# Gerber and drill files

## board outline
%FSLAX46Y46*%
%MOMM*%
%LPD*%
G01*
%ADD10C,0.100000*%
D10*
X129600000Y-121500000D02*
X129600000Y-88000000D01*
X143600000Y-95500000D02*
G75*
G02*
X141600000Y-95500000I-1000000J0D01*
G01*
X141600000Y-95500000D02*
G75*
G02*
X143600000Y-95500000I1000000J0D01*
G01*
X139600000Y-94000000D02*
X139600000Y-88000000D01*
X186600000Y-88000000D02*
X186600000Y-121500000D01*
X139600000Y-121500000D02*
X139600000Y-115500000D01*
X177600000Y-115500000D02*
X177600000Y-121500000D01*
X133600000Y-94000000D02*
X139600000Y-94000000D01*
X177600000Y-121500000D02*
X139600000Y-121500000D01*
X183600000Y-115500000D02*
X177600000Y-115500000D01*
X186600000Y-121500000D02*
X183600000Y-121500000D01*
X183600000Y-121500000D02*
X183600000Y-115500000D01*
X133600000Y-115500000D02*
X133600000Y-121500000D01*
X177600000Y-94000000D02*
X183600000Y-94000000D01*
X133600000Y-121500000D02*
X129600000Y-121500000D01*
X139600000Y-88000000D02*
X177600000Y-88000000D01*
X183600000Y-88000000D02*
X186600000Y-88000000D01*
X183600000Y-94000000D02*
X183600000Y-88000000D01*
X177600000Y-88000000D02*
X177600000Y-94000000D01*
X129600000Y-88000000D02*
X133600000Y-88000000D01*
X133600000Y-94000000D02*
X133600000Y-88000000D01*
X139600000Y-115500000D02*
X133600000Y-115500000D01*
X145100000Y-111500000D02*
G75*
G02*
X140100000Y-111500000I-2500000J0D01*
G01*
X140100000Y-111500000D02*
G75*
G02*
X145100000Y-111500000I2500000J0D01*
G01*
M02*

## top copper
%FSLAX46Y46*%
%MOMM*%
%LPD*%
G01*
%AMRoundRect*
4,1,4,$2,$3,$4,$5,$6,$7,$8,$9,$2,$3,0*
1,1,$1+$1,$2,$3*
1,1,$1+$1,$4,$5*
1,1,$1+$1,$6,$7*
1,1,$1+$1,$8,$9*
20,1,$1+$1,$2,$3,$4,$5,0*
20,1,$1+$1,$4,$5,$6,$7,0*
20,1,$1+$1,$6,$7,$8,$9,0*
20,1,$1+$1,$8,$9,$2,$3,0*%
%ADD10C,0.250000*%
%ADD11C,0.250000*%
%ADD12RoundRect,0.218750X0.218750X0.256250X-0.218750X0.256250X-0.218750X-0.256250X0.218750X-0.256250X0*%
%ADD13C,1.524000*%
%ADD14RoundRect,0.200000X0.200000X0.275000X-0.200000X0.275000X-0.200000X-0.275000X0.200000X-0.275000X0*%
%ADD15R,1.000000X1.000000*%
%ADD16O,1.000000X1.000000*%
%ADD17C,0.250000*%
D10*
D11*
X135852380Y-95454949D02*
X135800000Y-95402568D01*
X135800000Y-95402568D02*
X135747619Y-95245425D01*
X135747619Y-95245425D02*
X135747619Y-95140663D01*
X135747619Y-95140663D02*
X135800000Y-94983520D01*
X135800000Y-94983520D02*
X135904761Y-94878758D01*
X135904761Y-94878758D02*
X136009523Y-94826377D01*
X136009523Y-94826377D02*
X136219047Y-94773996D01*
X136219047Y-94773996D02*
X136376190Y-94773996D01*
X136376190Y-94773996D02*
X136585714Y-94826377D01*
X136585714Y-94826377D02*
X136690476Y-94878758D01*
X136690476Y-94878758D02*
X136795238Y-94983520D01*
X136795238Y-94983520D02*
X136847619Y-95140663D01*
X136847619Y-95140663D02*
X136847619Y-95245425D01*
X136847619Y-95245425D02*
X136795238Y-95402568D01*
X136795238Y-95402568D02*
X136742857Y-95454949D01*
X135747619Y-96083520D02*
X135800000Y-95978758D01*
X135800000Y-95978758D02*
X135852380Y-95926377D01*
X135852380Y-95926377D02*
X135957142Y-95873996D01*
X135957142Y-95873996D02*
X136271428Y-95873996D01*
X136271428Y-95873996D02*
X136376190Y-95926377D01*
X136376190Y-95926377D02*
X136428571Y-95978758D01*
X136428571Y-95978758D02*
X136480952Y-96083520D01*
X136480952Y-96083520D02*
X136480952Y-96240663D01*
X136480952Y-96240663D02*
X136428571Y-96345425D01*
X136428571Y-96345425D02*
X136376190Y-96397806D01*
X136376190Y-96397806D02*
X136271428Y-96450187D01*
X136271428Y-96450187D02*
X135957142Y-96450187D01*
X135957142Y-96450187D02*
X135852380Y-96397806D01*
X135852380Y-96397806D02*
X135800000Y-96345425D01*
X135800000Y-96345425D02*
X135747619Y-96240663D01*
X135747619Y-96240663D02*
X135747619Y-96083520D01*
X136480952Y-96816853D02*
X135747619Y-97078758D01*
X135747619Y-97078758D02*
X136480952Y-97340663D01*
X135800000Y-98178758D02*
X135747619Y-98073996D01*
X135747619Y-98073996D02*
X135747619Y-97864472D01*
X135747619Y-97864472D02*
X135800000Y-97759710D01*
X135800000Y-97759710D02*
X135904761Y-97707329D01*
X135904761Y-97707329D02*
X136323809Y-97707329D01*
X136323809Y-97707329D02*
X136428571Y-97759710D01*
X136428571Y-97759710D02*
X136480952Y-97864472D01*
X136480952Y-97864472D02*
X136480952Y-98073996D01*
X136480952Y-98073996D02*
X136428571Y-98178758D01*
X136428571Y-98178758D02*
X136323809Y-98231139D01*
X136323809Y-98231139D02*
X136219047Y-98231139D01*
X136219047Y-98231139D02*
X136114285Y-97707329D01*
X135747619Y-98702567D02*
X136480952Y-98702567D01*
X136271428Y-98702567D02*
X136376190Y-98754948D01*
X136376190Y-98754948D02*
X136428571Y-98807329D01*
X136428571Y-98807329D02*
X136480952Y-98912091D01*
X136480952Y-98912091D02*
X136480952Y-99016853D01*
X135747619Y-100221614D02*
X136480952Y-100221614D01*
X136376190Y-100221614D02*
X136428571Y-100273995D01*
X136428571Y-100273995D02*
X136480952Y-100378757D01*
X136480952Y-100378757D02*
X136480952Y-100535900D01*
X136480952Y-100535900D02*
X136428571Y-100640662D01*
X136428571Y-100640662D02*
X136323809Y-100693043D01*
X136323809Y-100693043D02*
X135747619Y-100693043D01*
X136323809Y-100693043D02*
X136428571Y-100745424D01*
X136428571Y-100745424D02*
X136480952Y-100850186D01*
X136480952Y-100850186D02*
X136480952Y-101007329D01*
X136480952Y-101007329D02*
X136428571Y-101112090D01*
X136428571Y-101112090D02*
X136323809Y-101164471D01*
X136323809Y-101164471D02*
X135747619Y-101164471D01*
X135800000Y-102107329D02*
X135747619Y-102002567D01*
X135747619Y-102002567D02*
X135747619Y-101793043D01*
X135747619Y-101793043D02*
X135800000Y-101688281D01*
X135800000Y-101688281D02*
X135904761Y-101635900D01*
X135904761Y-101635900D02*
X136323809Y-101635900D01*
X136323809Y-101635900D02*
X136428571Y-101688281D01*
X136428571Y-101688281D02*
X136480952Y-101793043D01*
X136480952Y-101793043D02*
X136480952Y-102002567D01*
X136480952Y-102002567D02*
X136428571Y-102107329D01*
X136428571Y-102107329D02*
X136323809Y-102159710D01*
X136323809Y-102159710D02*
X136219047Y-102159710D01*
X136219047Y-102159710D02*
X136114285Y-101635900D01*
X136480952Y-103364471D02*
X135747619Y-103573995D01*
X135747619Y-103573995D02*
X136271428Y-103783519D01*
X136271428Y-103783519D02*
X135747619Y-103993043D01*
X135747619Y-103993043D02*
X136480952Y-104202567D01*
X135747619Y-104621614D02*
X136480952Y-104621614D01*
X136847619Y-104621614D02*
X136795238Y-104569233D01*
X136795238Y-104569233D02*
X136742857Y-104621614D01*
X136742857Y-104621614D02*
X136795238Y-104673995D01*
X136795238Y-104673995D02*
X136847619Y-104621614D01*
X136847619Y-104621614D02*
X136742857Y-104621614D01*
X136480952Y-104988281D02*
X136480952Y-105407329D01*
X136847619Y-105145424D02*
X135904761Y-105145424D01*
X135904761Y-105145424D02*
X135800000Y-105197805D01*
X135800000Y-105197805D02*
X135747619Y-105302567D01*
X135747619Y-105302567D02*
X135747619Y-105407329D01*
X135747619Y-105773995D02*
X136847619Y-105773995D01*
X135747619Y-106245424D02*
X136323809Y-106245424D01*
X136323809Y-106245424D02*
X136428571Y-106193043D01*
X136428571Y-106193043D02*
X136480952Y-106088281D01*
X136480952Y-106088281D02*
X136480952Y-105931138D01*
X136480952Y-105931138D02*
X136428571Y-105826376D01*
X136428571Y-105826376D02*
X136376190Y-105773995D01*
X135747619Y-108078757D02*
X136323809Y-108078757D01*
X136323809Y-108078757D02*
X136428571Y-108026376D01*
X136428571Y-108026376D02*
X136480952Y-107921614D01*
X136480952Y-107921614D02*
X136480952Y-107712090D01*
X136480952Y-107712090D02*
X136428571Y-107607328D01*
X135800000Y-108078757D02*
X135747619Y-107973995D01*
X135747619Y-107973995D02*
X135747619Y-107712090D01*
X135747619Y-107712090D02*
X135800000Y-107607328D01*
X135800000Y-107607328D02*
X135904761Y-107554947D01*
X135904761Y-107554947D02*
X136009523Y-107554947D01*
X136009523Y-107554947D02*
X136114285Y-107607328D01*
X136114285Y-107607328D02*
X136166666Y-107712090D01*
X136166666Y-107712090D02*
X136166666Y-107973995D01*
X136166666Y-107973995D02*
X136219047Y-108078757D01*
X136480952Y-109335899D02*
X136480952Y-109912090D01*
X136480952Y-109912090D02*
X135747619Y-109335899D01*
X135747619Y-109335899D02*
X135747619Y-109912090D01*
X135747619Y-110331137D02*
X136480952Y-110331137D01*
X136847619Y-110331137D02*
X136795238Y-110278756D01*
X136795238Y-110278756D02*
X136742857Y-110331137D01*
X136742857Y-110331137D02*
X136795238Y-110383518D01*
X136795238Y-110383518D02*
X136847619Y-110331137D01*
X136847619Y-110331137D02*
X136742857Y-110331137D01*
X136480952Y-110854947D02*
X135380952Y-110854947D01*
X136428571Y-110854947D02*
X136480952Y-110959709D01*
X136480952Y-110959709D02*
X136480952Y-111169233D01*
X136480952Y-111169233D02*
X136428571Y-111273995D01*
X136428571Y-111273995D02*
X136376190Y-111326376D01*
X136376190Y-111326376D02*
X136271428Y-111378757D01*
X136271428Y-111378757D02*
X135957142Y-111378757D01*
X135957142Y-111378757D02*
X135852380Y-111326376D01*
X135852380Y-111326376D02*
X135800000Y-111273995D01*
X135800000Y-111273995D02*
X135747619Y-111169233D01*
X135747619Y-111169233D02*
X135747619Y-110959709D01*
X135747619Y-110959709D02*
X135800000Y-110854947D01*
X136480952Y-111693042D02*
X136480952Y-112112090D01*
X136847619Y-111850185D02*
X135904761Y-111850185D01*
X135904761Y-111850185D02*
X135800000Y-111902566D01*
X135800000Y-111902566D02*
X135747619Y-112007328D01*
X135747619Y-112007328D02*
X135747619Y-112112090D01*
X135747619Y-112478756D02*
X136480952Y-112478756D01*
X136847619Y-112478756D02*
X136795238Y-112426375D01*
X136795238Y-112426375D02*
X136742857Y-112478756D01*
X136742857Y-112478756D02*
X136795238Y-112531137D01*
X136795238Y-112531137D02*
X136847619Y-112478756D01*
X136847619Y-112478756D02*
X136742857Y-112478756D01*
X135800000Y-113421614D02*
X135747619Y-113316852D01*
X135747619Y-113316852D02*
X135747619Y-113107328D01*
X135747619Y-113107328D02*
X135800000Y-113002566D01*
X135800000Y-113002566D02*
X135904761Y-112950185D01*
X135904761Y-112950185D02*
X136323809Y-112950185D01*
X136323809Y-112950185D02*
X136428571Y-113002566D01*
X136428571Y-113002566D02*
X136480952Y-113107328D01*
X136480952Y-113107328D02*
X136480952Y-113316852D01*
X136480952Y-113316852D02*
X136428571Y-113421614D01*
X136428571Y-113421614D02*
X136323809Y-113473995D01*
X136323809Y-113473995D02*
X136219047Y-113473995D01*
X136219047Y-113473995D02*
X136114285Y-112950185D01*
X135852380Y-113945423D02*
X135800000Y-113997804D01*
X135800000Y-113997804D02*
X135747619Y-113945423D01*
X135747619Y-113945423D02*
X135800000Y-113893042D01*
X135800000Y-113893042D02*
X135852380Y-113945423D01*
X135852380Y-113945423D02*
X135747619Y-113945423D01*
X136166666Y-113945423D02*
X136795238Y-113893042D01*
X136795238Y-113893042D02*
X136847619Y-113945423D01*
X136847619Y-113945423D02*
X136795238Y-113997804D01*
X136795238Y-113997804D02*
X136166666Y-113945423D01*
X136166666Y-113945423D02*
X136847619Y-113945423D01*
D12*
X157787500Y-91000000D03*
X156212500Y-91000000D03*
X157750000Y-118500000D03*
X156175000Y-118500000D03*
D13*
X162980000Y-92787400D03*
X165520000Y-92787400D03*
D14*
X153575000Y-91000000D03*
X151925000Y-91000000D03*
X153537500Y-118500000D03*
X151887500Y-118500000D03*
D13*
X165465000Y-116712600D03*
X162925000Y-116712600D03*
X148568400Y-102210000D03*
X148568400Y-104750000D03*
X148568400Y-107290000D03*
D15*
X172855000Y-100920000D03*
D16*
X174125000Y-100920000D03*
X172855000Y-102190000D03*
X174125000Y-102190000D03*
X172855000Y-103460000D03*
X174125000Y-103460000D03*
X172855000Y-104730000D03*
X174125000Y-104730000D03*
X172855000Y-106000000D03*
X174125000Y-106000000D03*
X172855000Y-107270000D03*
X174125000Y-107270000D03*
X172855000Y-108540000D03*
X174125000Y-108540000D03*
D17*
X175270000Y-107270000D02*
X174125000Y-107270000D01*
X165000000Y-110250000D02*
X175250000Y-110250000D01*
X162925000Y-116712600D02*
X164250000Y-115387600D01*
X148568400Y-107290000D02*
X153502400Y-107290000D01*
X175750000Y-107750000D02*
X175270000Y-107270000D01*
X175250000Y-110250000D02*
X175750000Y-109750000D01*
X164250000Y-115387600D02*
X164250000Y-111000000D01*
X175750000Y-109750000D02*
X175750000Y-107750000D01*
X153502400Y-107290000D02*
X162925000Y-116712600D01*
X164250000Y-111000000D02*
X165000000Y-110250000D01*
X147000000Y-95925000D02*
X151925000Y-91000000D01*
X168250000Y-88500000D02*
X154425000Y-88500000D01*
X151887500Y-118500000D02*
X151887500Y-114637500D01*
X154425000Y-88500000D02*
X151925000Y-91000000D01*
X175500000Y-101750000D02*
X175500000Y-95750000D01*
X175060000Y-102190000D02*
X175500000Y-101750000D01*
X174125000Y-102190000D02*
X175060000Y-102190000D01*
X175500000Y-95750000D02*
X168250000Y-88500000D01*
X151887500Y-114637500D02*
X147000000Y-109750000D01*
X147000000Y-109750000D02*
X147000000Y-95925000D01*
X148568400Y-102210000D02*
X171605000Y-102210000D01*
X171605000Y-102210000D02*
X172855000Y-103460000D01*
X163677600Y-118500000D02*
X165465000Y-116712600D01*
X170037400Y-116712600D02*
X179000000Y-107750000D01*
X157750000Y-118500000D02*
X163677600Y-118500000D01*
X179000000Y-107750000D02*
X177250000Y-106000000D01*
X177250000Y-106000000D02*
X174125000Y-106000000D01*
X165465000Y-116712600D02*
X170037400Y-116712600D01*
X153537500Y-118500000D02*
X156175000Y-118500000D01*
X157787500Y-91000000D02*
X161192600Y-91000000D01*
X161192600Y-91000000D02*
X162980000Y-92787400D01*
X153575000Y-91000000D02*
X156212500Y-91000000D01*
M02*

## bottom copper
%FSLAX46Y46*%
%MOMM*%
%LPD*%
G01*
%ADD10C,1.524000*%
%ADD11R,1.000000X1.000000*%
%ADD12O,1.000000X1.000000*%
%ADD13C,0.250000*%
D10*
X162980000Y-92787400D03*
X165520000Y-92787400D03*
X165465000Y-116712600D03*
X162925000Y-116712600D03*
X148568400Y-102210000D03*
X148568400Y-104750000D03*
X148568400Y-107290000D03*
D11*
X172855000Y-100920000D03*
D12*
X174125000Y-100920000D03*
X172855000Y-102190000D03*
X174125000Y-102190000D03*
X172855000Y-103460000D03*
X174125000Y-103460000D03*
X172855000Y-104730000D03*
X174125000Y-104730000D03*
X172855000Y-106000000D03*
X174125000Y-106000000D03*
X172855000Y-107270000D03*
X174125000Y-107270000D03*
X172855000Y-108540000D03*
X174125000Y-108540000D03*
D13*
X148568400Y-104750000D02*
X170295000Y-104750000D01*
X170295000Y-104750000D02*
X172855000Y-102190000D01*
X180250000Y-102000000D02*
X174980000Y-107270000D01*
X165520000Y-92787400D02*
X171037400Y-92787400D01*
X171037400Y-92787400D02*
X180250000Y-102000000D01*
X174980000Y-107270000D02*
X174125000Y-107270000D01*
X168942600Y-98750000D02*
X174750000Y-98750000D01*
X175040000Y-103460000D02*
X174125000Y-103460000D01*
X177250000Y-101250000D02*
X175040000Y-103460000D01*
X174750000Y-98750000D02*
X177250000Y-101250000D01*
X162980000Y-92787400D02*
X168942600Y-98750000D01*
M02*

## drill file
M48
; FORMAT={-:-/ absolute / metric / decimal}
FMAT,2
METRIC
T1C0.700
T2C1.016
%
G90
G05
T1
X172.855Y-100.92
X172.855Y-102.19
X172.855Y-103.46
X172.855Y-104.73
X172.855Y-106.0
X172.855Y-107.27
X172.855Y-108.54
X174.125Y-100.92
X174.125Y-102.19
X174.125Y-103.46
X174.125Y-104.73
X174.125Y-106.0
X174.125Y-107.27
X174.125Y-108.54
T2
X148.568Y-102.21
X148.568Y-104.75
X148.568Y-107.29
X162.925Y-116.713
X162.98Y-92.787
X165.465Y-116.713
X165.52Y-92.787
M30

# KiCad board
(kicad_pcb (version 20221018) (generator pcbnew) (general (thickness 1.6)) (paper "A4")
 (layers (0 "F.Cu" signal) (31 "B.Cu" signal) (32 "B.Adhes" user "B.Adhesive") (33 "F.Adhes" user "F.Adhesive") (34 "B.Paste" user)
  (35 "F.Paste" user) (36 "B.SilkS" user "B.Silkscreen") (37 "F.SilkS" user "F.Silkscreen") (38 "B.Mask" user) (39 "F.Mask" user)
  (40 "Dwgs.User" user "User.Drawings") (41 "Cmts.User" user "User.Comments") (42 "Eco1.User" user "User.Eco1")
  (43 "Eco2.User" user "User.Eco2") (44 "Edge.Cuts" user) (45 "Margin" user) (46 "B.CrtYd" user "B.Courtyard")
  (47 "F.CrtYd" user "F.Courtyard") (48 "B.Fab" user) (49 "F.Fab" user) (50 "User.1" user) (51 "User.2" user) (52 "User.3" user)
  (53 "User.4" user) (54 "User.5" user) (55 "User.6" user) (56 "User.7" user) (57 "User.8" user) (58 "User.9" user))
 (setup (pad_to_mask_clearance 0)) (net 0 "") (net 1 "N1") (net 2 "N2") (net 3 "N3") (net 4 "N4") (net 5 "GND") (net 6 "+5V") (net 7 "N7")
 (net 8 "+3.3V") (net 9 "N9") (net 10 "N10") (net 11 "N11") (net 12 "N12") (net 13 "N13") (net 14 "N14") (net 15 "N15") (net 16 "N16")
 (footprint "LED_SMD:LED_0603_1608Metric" (layer "F.Cu") (at 157 91 180)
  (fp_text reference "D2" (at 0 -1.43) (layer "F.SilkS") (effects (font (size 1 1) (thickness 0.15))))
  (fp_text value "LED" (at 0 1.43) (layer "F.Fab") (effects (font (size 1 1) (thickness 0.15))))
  (pad "1" smd roundrect (at -0.7875 0 180) (size 0.875 0.95) (layers "F.Cu" "F.Paste" "F.Mask") (roundrect_rratio 0.25) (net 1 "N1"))
  (pad "2" smd roundrect (at 0.7875 0 180) (size 0.875 0.95) (layers "F.Cu" "F.Paste" "F.Mask") (roundrect_rratio 0.25) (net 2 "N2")))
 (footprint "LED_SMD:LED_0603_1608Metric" (layer "F.Cu") (at 156.9625 118.5 180)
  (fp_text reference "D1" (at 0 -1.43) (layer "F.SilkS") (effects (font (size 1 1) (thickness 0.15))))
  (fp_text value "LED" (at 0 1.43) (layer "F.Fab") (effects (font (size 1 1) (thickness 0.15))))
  (pad "1" smd roundrect (at -0.7875 0 180) (size 0.875 0.95) (layers "F.Cu" "F.Paste" "F.Mask") (roundrect_rratio 0.25) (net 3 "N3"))
  (pad "2" smd roundrect (at 0.7875 0 180) (size 0.875 0.95) (layers "F.Cu" "F.Paste" "F.Mask") (roundrect_rratio 0.25) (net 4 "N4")))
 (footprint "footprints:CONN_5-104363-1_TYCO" (layer "F.Cu") (at 162.98 92.7874)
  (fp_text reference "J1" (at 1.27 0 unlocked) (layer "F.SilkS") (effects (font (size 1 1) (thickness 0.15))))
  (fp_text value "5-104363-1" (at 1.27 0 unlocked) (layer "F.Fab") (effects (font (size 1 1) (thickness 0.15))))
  (pad "1" thru_hole circle (at 0 0) (size 1.524 1.524) (drill 1.016) (layers "*.Cu" "*.Mask") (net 1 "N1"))
  (pad "2" thru_hole circle (at 2.54 0) (size 1.524 1.524) (drill 1.016) (layers "*.Cu" "*.Mask") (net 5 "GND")))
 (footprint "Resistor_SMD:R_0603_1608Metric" (layer "F.Cu") (at 152.75 91 180)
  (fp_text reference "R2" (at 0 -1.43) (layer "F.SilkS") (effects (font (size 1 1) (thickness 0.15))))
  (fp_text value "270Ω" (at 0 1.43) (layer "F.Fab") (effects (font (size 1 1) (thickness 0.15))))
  (pad "1" smd roundrect (at -0.825 0 180) (size 0.8 0.95) (layers "F.Cu" "F.Paste" "F.Mask") (roundrect_rratio 0.25) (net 2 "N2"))
  (pad "2" smd roundrect (at 0.825 0 180) (size 0.8 0.95) (layers "F.Cu" "F.Paste" "F.Mask") (roundrect_rratio 0.25) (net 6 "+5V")))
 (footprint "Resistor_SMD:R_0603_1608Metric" (layer "F.Cu") (at 152.7125 118.5 180)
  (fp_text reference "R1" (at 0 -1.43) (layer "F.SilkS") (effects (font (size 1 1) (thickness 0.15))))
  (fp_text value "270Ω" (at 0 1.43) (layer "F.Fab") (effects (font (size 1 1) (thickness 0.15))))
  (pad "1" smd roundrect (at -0.825 0 180) (size 0.8 0.95) (layers "F.Cu" "F.Paste" "F.Mask") (roundrect_rratio 0.25) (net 4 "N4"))
  (pad "2" smd roundrect (at 0.825 0 180) (size 0.8 0.95) (layers "F.Cu" "F.Paste" "F.Mask") (roundrect_rratio 0.25) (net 6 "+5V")))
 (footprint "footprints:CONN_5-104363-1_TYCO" (layer "F.Cu") (at 165.465 116.7126 180)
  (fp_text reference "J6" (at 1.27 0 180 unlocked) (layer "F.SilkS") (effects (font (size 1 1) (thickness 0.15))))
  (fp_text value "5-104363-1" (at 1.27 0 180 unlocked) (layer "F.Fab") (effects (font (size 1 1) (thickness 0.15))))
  (pad "1" thru_hole circle (at 0 0 180) (size 1.524 1.524) (drill 1.016) (layers "*.Cu" "*.Mask") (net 3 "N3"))
  (pad "2" thru_hole circle (at 2.54 0 180) (size 1.524 1.524) (drill 1.016) (layers "*.Cu" "*.Mask") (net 5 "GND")))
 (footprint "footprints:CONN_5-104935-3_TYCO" (layer "F.Cu") (at 148.5684 102.21 -90)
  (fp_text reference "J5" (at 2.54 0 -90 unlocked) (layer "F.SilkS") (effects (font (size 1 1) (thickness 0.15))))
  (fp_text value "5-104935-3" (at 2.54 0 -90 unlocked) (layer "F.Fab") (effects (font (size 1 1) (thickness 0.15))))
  (pad "1" thru_hole circle (at 0 0 270) (size 1.524 1.524) (drill 1.016) (layers "*.Cu" "*.Mask") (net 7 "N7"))
  (pad "2" thru_hole circle (at 2.54 0 270) (size 1.524 1.524) (drill 1.016) (layers "*.Cu" "*.Mask") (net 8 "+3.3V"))
  (pad "3" thru_hole circle (at 5.08 0 270) (size 1.524 1.524) (drill 1.016) (layers "*.Cu" "*.Mask") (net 5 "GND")))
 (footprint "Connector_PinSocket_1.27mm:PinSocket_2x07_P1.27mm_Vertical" (layer "B.Cu") (at 172.855 100.92 180)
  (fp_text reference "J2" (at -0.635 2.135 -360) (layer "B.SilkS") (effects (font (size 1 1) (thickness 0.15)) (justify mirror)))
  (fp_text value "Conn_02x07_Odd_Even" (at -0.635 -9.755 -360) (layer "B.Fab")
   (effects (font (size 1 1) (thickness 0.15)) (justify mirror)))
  (pad "1" thru_hole rect (at 0 0 180) (size 1 1) (drill 0.7) (layers "*.Cu" "*.Mask") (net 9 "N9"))
  (pad "2" thru_hole oval (at -1.27 0 180) (size 1 1) (drill 0.7) (layers "*.Cu" "*.Mask") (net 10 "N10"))
  (pad "3" thru_hole oval (at 0 -1.27 180) (size 1 1) (drill 0.7) (layers "*.Cu" "*.Mask") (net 8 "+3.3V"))
  (pad "4" thru_hole oval (at -1.27 -1.27 180) (size 1 1) (drill 0.7) (layers "*.Cu" "*.Mask") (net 6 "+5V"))
  (pad "5" thru_hole oval (at 0 -2.54 180) (size 1 1) (drill 0.7) (layers "*.Cu" "*.Mask") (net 7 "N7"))
  (pad "6" thru_hole oval (at -1.27 -2.54 180) (size 1 1) (drill 0.7) (layers "*.Cu" "*.Mask") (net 1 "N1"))
  (pad "7" thru_hole oval (at 0 -3.81 180) (size 1 1) (drill 0.7) (layers "*.Cu" "*.Mask") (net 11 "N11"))
  (pad "8" thru_hole oval (at -1.27 -3.81 180) (size 1 1) (drill 0.7) (layers "*.Cu" "*.Mask") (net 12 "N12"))
  (pad "9" thru_hole oval (at 0 -5.08 180) (size 1 1) (drill 0.7) (layers "*.Cu" "*.Mask") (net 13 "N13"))
  (pad "10" thru_hole oval (at -1.27 -5.08 180) (size 1 1) (drill 0.7) (layers "*.Cu" "*.Mask") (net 3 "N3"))
  (pad "11" thru_hole oval (at 0 -6.35 180) (size 1 1) (drill 0.7) (layers "*.Cu" "*.Mask") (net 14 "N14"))
  (pad "12" thru_hole oval (at -1.27 -6.35 180) (size 1 1) (drill 0.7) (layers "*.Cu" "*.Mask") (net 5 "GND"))
  (pad "13" thru_hole oval (at 0 -7.62 180) (size 1 1) (drill 0.7) (layers "*.Cu" "*.Mask") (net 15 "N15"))
  (pad "14" thru_hole oval (at -1.27 -7.62 180) (size 1 1) (drill 0.7) (layers "*.Cu" "*.Mask") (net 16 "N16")))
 (gr_line (start 129.6 121.5) (end 129.6 88) (stroke (width 0.1) (type default)) (layer "Edge.Cuts"))
 (gr_circle (center 142.6 95.5) (end 141.6 95.5) (stroke (width 0.1) (type default)) (fill none) (layer "Edge.Cuts"))
 (gr_line (start 139.6 94) (end 139.6 88) (stroke (width 0.1) (type default)) (layer "Edge.Cuts"))
 (gr_line (start 186.6 88) (end 186.6 121.5) (stroke (width 0.1) (type default)) (layer "Edge.Cuts"))
 (gr_line (start 139.6 121.5) (end 139.6 115.5) (stroke (width 0.1) (type default)) (layer "Edge.Cuts"))
 (gr_line (start 177.6 115.5) (end 177.6 121.5) (stroke (width 0.1) (type default)) (layer "Edge.Cuts"))
 (gr_line (start 133.6 94) (end 139.6 94) (stroke (width 0.1) (type default)) (layer "Edge.Cuts"))
 (gr_line (start 177.6 121.5) (end 139.6 121.5) (stroke (width 0.1) (type default)) (layer "Edge.Cuts"))
 (gr_line (start 183.6 115.5) (end 177.6 115.5) (stroke (width 0.1) (type default)) (layer "Edge.Cuts"))
 (gr_line (start 186.6 121.5) (end 183.6 121.5) (stroke (width 0.1) (type default)) (layer "Edge.Cuts"))
 (gr_line (start 183.6 121.5) (end 183.6 115.5) (stroke (width 0.1) (type default)) (layer "Edge.Cuts"))
 (gr_line (start 133.6 115.5) (end 133.6 121.5) (stroke (width 0.1) (type default)) (layer "Edge.Cuts"))
 (gr_line (start 177.6 94) (end 183.6 94) (stroke (width 0.1) (type default)) (layer "Edge.Cuts"))
 (gr_line (start 133.6 121.5) (end 129.6 121.5) (stroke (width 0.1) (type default)) (layer "Edge.Cuts"))
 (gr_line (start 139.6 88) (end 177.6 88) (stroke (width 0.1) (type default)) (layer "Edge.Cuts"))
 (gr_line (start 183.6 88) (end 186.6 88) (stroke (width 0.1) (type default)) (layer "Edge.Cuts"))
 (gr_line (start 183.6 94) (end 183.6 88) (stroke (width 0.1) (type default)) (layer "Edge.Cuts"))
 (gr_line (start 177.6 88) (end 177.6 94) (stroke (width 0.1) (type default)) (layer "Edge.Cuts"))
 (gr_line (start 129.6 88) (end 133.6 88) (stroke (width 0.1) (type default)) (layer "Edge.Cuts"))
 (gr_line (start 133.6 94) (end 133.6 88) (stroke (width 0.1) (type default)) (layer "Edge.Cuts"))
 (gr_line (start 139.6 115.5) (end 133.6 115.5) (stroke (width 0.1) (type default)) (layer "Edge.Cuts"))
 (gr_circle (center 142.6 111.5) (end 140.1 111.5) (stroke (width 0.1) (type default)) (fill none) (layer "Edge.Cuts"))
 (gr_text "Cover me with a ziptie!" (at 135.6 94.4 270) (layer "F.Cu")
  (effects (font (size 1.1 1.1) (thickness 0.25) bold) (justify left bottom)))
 (segment (start 148.5684 104.75) (end 170.295 104.75) (width 0.25) (layer "B.Cu") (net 8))
 (segment (start 170.295 104.75) (end 172.855 102.19) (width 0.25) (layer "B.Cu") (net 8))
 (segment (start 175.27 107.27) (end 174.125 107.27) (width 0.25) (layer "F.Cu") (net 5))
 (segment (start 165 110.25) (end 175.25 110.25) (width 0.25) (layer "F.Cu") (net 5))
 (segment (start 162.925 116.7126) (end 164.25 115.3876) (width 0.25) (layer "F.Cu") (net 5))
 (segment (start 148.5684 107.29) (end 153.5024 107.29) (width 0.25) (layer "F.Cu") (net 5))
 (segment (start 175.75 107.75) (end 175.27 107.27) (width 0.25) (layer "F.Cu") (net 5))
 (segment (start 175.25 110.25) (end 175.75 109.75) (width 0.25) (layer "F.Cu") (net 5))
 (segment (start 164.25 115.3876) (end 164.25 111) (width 0.25) (layer "F.Cu") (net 5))
 (segment (start 175.75 109.75) (end 175.75 107.75) (width 0.25) (layer "F.Cu") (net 5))
 (segment (start 153.5024 107.29) (end 162.925 116.7126) (width 0.25) (layer "F.Cu") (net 5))
 (segment (start 164.25 111) (end 165 110.25) (width 0.25) (layer "F.Cu") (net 5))
 (segment (start 180.25 102) (end 174.98 107.27) (width 0.25) (layer "B.Cu") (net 5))
 (segment (start 165.52 92.7874) (end 171.0374 92.7874) (width 0.25) (layer "B.Cu") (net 5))
 (segment (start 171.0374 92.7874) (end 180.25 102) (width 0.25) (layer "B.Cu") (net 5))
 (segment (start 174.98 107.27) (end 174.125 107.27) (width 0.25) (layer "B.Cu") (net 5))
 (segment (start 147 95.925) (end 151.925 91) (width 0.25) (layer "F.Cu") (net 6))
 (segment (start 168.25 88.5) (end 154.425 88.5) (width 0.25) (layer "F.Cu") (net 6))
 (segment (start 151.8875 118.5) (end 151.8875 114.6375) (width 0.25) (layer "F.Cu") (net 6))
 (segment (start 154.425 88.5) (end 151.925 91) (width 0.25) (layer "F.Cu") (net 6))
 (segment (start 175.5 101.75) (end 175.5 95.75) (width 0.25) (layer "F.Cu") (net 6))
 (segment (start 175.06 102.19) (end 175.5 101.75) (width 0.25) (layer "F.Cu") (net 6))
 (segment (start 174.125 102.19) (end 175.06 102.19) (width 0.25) (layer "F.Cu") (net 6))
 (segment (start 175.5 95.75) (end 168.25 88.5) (width 0.25) (layer "F.Cu") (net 6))
 (segment (start 151.8875 114.6375) (end 147 109.75) (width 0.25) (layer "F.Cu") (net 6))
 (segment (start 147 109.75) (end 147 95.925) (width 0.25) (layer "F.Cu") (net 6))
 (segment (start 148.5684 102.21) (end 171.605 102.21) (width 0.25) (layer "F.Cu") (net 7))
 (segment (start 171.605 102.21) (end 172.855 103.46) (width 0.25) (layer "F.Cu") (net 7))
 (segment (start 163.6776 118.5) (end 165.465 116.7126) (width 0.25) (layer "F.Cu") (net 3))
 (segment (start 170.0374 116.7126) (end 179 107.75) (width 0.25) (layer "F.Cu") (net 3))
 (segment (start 157.75 118.5) (end 163.6776 118.5) (width 0.25) (layer "F.Cu") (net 3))
 (segment (start 179 107.75) (end 177.25 106) (width 0.25) (layer "F.Cu") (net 3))
 (segment (start 177.25 106) (end 174.125 106) (width 0.25) (layer "F.Cu") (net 3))
 (segment (start 165.465 116.7126) (end 170.0374 116.7126) (width 0.25) (layer "F.Cu") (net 3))
 (segment (start 153.5375 118.5) (end 156.175 118.5) (width 0.25) (layer "F.Cu") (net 4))
 (segment (start 157.7875 91) (end 161.1926 91) (width 0.25) (layer "F.Cu") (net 1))
 (segment (start 161.1926 91) (end 162.98 92.7874) (width 0.25) (layer "F.Cu") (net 1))
 (segment (start 168.9426 98.75) (end 174.75 98.75) (width 0.25) (layer "B.Cu") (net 1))
 (segment (start 175.04 103.46) (end 174.125 103.46) (width 0.25) (layer "B.Cu") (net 1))
 (segment (start 177.25 101.25) (end 175.04 103.46) (width 0.25) (layer "B.Cu") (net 1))
 (segment (start 174.75 98.75) (end 177.25 101.25) (width 0.25) (layer "B.Cu") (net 1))
 (segment (start 162.98 92.7874) (end 168.9426 98.75) (width 0.25) (layer "B.Cu") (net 1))
 (segment (start 153.575 91) (end 156.2125 91) (width 0.25) (layer "F.Cu") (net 2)))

